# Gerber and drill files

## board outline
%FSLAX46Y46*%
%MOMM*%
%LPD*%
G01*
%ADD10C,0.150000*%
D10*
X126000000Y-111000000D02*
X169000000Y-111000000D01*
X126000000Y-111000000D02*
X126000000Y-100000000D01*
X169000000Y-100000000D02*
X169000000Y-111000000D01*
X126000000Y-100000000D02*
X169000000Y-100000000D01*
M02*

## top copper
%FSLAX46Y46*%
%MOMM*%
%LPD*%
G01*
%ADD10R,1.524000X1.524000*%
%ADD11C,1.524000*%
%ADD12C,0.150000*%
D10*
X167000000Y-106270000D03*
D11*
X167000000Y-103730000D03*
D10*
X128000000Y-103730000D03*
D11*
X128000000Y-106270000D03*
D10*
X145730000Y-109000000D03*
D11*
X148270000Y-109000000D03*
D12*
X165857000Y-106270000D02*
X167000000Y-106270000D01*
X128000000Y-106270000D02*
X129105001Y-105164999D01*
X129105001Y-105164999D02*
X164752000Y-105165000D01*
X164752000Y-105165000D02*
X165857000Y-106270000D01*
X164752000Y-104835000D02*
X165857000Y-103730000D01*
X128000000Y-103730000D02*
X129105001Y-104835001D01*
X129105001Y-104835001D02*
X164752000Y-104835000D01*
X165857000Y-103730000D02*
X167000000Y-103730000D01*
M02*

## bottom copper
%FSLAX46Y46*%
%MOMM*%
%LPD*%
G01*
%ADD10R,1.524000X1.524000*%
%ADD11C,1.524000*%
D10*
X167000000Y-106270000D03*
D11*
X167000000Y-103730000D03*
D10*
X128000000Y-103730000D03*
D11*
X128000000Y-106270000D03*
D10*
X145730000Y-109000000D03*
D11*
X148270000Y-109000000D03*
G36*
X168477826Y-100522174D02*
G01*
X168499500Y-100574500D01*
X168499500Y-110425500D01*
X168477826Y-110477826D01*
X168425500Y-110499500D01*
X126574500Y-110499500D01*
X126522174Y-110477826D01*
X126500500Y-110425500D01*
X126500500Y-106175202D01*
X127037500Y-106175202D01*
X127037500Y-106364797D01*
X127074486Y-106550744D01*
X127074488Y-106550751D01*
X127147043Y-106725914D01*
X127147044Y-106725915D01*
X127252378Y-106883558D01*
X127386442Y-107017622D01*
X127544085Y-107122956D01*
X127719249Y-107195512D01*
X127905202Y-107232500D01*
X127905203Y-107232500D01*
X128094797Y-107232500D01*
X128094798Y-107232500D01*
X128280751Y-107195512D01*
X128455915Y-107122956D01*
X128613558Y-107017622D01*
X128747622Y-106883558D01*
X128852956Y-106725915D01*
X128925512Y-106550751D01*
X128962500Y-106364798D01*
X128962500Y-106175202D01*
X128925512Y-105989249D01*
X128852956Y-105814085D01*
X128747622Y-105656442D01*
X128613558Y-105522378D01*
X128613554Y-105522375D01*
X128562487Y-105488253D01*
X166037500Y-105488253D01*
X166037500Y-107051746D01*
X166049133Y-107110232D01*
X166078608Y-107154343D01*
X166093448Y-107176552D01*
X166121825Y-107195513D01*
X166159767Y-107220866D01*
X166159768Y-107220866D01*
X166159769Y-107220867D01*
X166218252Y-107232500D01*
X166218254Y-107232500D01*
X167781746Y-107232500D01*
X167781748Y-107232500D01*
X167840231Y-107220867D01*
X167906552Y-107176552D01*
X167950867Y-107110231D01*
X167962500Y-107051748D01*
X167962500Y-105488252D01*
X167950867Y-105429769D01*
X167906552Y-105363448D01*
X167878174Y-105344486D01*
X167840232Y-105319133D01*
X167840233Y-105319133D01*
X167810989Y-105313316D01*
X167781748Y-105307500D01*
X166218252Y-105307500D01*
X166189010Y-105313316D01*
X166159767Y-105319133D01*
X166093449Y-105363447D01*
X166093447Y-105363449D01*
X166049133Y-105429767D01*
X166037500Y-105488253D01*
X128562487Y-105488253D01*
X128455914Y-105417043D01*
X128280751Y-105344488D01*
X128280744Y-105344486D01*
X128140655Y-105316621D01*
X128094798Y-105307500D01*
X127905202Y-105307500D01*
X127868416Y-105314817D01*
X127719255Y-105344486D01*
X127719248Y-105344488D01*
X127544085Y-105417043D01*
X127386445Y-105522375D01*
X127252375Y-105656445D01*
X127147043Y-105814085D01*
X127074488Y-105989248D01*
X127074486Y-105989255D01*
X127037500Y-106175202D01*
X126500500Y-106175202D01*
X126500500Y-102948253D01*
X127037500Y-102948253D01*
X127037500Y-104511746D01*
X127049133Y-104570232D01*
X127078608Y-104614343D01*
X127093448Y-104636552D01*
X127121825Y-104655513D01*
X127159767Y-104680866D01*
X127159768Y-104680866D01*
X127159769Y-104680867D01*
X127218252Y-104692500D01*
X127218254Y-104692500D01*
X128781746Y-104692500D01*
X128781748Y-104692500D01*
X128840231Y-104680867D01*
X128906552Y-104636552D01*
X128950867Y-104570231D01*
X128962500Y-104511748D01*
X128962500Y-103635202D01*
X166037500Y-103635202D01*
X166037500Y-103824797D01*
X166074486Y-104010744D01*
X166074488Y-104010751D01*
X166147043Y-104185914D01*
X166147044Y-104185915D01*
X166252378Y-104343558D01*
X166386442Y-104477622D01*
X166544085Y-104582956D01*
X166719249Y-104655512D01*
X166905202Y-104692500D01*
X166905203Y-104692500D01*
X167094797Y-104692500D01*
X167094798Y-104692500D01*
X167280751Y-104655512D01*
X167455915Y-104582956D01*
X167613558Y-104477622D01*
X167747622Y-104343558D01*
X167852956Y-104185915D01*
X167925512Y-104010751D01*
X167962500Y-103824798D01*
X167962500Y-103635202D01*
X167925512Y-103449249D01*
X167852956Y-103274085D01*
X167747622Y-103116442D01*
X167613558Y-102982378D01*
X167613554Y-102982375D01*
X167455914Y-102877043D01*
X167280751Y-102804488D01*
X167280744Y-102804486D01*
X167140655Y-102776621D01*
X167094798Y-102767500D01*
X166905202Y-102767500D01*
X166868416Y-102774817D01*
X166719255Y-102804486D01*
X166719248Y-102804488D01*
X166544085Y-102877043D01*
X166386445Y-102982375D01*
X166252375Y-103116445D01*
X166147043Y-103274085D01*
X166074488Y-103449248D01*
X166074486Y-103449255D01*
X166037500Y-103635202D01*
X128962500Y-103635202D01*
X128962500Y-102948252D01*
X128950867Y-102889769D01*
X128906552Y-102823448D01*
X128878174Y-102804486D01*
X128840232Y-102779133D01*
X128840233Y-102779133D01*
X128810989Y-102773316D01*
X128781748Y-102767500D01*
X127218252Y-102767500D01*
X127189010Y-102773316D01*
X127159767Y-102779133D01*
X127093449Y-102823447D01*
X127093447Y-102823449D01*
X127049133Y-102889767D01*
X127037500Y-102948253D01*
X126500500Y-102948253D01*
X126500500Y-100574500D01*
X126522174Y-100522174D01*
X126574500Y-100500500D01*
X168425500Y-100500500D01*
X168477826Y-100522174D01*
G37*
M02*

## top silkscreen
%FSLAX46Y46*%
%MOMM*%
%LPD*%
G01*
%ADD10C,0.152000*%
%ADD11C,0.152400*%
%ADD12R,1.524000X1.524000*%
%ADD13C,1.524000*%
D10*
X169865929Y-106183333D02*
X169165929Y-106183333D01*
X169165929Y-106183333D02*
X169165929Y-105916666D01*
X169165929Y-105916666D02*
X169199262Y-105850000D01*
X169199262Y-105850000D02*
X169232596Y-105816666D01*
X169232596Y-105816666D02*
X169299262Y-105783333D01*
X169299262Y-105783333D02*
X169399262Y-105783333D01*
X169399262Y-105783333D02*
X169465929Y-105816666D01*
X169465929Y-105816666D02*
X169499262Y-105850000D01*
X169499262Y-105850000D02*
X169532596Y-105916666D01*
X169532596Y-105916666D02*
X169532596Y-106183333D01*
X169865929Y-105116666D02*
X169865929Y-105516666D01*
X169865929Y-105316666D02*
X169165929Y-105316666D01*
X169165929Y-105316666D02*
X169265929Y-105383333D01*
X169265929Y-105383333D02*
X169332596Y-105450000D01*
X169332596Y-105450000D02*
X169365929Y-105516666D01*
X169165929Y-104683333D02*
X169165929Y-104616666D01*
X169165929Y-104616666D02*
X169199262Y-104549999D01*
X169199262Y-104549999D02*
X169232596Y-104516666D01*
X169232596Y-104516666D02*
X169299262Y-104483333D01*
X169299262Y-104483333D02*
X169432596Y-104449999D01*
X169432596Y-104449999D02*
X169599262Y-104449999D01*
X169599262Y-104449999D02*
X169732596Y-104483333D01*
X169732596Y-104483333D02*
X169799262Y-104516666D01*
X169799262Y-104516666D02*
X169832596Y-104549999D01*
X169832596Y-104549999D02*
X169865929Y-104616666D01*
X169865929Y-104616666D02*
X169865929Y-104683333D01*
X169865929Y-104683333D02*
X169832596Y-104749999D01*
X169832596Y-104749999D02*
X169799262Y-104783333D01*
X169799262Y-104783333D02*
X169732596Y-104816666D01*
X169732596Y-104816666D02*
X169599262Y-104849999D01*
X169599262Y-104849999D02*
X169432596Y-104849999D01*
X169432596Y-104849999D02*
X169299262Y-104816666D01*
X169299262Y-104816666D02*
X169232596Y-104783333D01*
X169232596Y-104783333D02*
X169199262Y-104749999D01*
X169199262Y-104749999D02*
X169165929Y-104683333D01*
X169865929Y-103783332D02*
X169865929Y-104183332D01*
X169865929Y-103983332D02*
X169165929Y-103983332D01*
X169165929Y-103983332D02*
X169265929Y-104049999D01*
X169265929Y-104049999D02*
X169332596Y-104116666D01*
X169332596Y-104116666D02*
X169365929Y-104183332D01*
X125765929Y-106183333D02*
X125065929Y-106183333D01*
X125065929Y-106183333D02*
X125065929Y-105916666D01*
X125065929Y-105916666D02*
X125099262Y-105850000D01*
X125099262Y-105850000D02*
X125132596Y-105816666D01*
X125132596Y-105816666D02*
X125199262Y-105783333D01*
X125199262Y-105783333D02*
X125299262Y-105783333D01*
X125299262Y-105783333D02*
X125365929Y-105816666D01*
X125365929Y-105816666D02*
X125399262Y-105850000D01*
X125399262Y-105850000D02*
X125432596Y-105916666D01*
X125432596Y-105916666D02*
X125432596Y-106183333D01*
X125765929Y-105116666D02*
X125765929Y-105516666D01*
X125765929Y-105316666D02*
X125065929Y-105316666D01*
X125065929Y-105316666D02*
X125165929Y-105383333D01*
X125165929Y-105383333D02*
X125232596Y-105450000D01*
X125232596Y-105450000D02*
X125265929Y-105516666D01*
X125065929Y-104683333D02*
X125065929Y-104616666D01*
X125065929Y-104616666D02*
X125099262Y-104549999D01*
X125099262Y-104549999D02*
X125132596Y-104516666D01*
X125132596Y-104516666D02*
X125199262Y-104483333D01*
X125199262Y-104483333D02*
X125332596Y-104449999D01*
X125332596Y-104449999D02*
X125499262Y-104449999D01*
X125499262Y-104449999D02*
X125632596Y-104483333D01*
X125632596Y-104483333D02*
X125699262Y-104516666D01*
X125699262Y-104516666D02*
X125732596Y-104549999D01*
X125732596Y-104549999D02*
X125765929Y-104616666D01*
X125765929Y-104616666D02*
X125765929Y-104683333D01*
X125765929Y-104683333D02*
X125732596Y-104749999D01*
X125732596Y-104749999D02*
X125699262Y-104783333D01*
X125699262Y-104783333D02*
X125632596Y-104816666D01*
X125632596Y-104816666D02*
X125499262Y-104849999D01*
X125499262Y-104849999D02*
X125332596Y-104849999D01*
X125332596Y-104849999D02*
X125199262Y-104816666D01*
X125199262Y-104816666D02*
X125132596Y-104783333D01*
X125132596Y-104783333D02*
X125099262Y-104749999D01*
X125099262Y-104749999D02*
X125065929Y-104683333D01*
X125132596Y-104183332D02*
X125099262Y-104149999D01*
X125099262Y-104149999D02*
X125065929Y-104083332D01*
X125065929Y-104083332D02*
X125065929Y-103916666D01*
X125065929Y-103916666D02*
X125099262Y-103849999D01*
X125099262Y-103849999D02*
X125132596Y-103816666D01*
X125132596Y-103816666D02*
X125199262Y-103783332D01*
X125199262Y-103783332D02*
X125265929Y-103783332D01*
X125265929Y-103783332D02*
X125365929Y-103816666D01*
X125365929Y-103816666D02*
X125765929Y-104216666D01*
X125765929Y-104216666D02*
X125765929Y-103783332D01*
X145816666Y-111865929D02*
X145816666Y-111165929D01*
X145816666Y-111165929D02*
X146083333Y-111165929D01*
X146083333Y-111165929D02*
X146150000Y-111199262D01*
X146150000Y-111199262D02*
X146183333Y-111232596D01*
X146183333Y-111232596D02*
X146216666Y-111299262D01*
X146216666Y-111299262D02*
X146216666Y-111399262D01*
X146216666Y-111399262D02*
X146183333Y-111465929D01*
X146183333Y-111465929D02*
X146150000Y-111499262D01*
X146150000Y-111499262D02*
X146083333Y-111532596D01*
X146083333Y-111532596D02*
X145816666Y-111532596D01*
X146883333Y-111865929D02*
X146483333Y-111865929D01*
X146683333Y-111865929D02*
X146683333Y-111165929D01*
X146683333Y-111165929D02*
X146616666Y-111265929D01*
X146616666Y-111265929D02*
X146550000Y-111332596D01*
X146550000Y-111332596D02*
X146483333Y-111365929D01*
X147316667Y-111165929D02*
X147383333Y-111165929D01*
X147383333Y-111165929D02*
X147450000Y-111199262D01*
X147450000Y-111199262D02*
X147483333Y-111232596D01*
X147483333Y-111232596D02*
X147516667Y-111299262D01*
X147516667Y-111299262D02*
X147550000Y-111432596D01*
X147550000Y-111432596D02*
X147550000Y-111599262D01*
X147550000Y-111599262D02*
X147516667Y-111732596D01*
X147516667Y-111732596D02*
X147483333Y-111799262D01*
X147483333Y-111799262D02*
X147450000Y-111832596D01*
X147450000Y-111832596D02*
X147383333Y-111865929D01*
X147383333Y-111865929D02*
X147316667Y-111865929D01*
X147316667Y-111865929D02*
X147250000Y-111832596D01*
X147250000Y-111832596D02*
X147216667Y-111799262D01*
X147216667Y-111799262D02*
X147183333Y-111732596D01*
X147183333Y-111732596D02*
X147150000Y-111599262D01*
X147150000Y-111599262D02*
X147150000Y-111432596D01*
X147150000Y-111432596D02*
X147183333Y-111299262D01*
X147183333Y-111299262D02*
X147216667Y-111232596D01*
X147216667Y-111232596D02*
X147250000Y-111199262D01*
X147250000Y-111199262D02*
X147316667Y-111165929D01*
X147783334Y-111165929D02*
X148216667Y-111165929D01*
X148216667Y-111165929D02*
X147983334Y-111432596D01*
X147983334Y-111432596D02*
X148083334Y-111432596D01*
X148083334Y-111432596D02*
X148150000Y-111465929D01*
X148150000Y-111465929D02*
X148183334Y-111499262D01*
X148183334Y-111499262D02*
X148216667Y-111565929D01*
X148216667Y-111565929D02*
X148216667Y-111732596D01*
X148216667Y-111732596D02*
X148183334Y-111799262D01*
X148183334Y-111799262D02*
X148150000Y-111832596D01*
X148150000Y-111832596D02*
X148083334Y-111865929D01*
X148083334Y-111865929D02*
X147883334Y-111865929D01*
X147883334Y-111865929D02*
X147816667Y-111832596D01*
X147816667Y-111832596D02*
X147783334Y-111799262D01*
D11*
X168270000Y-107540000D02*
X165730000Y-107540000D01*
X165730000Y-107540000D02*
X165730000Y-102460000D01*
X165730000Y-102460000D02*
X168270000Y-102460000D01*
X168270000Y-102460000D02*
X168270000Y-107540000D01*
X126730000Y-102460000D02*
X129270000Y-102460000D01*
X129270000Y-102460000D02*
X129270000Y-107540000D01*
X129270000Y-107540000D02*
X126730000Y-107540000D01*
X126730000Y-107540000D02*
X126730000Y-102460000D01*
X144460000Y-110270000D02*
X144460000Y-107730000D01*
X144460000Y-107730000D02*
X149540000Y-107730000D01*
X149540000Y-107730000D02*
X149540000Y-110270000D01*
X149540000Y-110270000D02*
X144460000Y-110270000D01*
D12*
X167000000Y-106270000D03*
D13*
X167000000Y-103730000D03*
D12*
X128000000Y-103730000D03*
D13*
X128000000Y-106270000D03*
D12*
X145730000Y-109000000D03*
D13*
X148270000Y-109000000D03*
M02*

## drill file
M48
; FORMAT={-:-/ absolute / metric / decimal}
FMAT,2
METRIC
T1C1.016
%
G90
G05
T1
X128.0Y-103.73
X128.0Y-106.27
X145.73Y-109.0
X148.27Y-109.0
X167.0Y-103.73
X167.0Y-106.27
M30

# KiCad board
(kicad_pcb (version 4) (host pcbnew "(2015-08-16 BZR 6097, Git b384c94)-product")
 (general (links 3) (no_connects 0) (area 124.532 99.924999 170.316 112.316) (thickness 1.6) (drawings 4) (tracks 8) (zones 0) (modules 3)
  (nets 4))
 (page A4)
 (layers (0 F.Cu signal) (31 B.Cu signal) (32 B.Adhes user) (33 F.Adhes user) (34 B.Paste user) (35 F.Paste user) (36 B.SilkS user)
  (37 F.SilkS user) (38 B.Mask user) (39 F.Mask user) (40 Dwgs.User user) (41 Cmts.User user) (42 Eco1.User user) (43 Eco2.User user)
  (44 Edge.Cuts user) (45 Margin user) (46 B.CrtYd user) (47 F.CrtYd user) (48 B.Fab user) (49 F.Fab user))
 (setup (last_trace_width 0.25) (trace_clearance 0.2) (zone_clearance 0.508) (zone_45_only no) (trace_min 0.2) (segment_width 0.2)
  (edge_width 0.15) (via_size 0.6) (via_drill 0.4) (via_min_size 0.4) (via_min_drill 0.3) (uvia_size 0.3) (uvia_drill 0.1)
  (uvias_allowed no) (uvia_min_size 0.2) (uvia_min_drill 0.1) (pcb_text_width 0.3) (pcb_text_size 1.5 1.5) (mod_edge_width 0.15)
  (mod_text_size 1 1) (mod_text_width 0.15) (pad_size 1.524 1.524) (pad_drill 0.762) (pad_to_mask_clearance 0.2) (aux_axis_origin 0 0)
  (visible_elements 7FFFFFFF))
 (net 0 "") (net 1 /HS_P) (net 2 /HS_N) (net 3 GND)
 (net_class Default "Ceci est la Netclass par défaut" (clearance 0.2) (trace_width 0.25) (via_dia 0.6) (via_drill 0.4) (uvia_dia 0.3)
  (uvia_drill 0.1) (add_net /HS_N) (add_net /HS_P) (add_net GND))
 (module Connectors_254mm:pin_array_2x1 (layer F.Cu) (at 167 105 90)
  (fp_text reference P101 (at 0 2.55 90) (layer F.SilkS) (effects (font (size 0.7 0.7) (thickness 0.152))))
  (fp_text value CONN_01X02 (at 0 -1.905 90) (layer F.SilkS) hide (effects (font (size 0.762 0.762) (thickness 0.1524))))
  (fp_line (start -2.54 1.27) (end -2.54 -1.27) (layer F.SilkS) (width 0.1524))
  (fp_line (start -2.54 -1.27) (end 2.54 -1.27) (layer F.SilkS) (width 0.1524))
  (fp_line (start 2.54 -1.27) (end 2.54 1.27) (layer F.SilkS) (width 0.1524))
  (fp_line (start 2.54 1.27) (end -2.54 1.27) (layer F.SilkS) (width 0.1524))
  (pad 1 thru_hole rect (at -1.27 0 90) (size 1.524 1.524) (drill 1.016) (layers *.Cu *.Mask F.SilkS) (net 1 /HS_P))
  (pad 2 thru_hole circle (at 1.27 0 90) (size 1.524 1.524) (drill 1.016) (layers *.Cu *.Mask F.SilkS) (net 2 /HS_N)))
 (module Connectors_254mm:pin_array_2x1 (layer F.Cu) (at 128 105 270)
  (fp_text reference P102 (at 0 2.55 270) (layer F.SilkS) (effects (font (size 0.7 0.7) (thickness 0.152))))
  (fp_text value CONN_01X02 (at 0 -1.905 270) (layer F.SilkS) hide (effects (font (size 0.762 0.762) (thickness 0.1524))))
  (fp_line (start -2.54 1.27) (end -2.54 -1.27) (layer F.SilkS) (width 0.1524))
  (fp_line (start -2.54 -1.27) (end 2.54 -1.27) (layer F.SilkS) (width 0.1524))
  (fp_line (start 2.54 -1.27) (end 2.54 1.27) (layer F.SilkS) (width 0.1524))
  (fp_line (start 2.54 1.27) (end -2.54 1.27) (layer F.SilkS) (width 0.1524))
  (pad 1 thru_hole rect (at -1.27 0 270) (size 1.524 1.524) (drill 1.016) (layers *.Cu *.Mask F.SilkS) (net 2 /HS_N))
  (pad 2 thru_hole circle (at 1.27 0 270) (size 1.524 1.524) (drill 1.016) (layers *.Cu *.Mask F.SilkS) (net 1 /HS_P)))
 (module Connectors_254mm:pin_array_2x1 (layer F.Cu) (at 147 109)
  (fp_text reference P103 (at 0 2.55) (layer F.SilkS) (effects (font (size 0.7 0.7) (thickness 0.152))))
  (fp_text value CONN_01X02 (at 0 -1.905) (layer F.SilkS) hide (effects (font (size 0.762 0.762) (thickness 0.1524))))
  (fp_line (start -2.54 1.27) (end -2.54 -1.27) (layer F.SilkS) (width 0.1524))
  (fp_line (start -2.54 -1.27) (end 2.54 -1.27) (layer F.SilkS) (width 0.1524))
  (fp_line (start 2.54 -1.27) (end 2.54 1.27) (layer F.SilkS) (width 0.1524))
  (fp_line (start 2.54 1.27) (end -2.54 1.27) (layer F.SilkS) (width 0.1524))
  (pad 1 thru_hole rect (at -1.27 0) (size 1.524 1.524) (drill 1.016) (layers *.Cu *.Mask F.SilkS) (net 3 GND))
  (pad 2 thru_hole circle (at 1.27 0) (size 1.524 1.524) (drill 1.016) (layers *.Cu *.Mask F.SilkS) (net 3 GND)))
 (gr_line (start 126 111) (end 169 111) (layer Edge.Cuts) (width 0.15))
 (gr_line (start 126 111) (end 126 100) (layer Edge.Cuts) (width 0.15))
 (gr_line (start 169 100) (end 169 111) (layer Edge.Cuts) (width 0.15))
 (gr_line (start 126 100) (end 169 100) (layer Edge.Cuts) (width 0.15))
 (segment (start 165.857 106.27) (end 167 106.27) (width 0.15) (layer F.Cu) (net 1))
 (segment (start 128 106.27) (end 129.105001 105.164999) (width 0.15) (layer F.Cu) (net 1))
 (segment (start 129.105001 105.164999) (end 164.752 105.165) (width 0.15) (layer F.Cu) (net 1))
 (segment (start 164.752 105.165) (end 165.857 106.27) (width 0.15) (layer F.Cu) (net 1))
 (segment (start 164.752 104.835) (end 165.857 103.73) (width 0.15) (layer F.Cu) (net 2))
 (segment (start 128 103.73) (end 129.105001 104.835001) (width 0.15) (layer F.Cu) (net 2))
 (segment (start 129.105001 104.835001) (end 164.752 104.835) (width 0.15) (layer F.Cu) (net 2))
 (segment (start 165.857 103.73) (end 167 103.73) (width 0.15) (layer F.Cu) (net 2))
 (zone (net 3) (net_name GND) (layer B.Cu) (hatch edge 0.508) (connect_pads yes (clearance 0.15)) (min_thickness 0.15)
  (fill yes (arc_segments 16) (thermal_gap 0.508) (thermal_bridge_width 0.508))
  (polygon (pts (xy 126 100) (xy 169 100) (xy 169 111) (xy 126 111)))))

